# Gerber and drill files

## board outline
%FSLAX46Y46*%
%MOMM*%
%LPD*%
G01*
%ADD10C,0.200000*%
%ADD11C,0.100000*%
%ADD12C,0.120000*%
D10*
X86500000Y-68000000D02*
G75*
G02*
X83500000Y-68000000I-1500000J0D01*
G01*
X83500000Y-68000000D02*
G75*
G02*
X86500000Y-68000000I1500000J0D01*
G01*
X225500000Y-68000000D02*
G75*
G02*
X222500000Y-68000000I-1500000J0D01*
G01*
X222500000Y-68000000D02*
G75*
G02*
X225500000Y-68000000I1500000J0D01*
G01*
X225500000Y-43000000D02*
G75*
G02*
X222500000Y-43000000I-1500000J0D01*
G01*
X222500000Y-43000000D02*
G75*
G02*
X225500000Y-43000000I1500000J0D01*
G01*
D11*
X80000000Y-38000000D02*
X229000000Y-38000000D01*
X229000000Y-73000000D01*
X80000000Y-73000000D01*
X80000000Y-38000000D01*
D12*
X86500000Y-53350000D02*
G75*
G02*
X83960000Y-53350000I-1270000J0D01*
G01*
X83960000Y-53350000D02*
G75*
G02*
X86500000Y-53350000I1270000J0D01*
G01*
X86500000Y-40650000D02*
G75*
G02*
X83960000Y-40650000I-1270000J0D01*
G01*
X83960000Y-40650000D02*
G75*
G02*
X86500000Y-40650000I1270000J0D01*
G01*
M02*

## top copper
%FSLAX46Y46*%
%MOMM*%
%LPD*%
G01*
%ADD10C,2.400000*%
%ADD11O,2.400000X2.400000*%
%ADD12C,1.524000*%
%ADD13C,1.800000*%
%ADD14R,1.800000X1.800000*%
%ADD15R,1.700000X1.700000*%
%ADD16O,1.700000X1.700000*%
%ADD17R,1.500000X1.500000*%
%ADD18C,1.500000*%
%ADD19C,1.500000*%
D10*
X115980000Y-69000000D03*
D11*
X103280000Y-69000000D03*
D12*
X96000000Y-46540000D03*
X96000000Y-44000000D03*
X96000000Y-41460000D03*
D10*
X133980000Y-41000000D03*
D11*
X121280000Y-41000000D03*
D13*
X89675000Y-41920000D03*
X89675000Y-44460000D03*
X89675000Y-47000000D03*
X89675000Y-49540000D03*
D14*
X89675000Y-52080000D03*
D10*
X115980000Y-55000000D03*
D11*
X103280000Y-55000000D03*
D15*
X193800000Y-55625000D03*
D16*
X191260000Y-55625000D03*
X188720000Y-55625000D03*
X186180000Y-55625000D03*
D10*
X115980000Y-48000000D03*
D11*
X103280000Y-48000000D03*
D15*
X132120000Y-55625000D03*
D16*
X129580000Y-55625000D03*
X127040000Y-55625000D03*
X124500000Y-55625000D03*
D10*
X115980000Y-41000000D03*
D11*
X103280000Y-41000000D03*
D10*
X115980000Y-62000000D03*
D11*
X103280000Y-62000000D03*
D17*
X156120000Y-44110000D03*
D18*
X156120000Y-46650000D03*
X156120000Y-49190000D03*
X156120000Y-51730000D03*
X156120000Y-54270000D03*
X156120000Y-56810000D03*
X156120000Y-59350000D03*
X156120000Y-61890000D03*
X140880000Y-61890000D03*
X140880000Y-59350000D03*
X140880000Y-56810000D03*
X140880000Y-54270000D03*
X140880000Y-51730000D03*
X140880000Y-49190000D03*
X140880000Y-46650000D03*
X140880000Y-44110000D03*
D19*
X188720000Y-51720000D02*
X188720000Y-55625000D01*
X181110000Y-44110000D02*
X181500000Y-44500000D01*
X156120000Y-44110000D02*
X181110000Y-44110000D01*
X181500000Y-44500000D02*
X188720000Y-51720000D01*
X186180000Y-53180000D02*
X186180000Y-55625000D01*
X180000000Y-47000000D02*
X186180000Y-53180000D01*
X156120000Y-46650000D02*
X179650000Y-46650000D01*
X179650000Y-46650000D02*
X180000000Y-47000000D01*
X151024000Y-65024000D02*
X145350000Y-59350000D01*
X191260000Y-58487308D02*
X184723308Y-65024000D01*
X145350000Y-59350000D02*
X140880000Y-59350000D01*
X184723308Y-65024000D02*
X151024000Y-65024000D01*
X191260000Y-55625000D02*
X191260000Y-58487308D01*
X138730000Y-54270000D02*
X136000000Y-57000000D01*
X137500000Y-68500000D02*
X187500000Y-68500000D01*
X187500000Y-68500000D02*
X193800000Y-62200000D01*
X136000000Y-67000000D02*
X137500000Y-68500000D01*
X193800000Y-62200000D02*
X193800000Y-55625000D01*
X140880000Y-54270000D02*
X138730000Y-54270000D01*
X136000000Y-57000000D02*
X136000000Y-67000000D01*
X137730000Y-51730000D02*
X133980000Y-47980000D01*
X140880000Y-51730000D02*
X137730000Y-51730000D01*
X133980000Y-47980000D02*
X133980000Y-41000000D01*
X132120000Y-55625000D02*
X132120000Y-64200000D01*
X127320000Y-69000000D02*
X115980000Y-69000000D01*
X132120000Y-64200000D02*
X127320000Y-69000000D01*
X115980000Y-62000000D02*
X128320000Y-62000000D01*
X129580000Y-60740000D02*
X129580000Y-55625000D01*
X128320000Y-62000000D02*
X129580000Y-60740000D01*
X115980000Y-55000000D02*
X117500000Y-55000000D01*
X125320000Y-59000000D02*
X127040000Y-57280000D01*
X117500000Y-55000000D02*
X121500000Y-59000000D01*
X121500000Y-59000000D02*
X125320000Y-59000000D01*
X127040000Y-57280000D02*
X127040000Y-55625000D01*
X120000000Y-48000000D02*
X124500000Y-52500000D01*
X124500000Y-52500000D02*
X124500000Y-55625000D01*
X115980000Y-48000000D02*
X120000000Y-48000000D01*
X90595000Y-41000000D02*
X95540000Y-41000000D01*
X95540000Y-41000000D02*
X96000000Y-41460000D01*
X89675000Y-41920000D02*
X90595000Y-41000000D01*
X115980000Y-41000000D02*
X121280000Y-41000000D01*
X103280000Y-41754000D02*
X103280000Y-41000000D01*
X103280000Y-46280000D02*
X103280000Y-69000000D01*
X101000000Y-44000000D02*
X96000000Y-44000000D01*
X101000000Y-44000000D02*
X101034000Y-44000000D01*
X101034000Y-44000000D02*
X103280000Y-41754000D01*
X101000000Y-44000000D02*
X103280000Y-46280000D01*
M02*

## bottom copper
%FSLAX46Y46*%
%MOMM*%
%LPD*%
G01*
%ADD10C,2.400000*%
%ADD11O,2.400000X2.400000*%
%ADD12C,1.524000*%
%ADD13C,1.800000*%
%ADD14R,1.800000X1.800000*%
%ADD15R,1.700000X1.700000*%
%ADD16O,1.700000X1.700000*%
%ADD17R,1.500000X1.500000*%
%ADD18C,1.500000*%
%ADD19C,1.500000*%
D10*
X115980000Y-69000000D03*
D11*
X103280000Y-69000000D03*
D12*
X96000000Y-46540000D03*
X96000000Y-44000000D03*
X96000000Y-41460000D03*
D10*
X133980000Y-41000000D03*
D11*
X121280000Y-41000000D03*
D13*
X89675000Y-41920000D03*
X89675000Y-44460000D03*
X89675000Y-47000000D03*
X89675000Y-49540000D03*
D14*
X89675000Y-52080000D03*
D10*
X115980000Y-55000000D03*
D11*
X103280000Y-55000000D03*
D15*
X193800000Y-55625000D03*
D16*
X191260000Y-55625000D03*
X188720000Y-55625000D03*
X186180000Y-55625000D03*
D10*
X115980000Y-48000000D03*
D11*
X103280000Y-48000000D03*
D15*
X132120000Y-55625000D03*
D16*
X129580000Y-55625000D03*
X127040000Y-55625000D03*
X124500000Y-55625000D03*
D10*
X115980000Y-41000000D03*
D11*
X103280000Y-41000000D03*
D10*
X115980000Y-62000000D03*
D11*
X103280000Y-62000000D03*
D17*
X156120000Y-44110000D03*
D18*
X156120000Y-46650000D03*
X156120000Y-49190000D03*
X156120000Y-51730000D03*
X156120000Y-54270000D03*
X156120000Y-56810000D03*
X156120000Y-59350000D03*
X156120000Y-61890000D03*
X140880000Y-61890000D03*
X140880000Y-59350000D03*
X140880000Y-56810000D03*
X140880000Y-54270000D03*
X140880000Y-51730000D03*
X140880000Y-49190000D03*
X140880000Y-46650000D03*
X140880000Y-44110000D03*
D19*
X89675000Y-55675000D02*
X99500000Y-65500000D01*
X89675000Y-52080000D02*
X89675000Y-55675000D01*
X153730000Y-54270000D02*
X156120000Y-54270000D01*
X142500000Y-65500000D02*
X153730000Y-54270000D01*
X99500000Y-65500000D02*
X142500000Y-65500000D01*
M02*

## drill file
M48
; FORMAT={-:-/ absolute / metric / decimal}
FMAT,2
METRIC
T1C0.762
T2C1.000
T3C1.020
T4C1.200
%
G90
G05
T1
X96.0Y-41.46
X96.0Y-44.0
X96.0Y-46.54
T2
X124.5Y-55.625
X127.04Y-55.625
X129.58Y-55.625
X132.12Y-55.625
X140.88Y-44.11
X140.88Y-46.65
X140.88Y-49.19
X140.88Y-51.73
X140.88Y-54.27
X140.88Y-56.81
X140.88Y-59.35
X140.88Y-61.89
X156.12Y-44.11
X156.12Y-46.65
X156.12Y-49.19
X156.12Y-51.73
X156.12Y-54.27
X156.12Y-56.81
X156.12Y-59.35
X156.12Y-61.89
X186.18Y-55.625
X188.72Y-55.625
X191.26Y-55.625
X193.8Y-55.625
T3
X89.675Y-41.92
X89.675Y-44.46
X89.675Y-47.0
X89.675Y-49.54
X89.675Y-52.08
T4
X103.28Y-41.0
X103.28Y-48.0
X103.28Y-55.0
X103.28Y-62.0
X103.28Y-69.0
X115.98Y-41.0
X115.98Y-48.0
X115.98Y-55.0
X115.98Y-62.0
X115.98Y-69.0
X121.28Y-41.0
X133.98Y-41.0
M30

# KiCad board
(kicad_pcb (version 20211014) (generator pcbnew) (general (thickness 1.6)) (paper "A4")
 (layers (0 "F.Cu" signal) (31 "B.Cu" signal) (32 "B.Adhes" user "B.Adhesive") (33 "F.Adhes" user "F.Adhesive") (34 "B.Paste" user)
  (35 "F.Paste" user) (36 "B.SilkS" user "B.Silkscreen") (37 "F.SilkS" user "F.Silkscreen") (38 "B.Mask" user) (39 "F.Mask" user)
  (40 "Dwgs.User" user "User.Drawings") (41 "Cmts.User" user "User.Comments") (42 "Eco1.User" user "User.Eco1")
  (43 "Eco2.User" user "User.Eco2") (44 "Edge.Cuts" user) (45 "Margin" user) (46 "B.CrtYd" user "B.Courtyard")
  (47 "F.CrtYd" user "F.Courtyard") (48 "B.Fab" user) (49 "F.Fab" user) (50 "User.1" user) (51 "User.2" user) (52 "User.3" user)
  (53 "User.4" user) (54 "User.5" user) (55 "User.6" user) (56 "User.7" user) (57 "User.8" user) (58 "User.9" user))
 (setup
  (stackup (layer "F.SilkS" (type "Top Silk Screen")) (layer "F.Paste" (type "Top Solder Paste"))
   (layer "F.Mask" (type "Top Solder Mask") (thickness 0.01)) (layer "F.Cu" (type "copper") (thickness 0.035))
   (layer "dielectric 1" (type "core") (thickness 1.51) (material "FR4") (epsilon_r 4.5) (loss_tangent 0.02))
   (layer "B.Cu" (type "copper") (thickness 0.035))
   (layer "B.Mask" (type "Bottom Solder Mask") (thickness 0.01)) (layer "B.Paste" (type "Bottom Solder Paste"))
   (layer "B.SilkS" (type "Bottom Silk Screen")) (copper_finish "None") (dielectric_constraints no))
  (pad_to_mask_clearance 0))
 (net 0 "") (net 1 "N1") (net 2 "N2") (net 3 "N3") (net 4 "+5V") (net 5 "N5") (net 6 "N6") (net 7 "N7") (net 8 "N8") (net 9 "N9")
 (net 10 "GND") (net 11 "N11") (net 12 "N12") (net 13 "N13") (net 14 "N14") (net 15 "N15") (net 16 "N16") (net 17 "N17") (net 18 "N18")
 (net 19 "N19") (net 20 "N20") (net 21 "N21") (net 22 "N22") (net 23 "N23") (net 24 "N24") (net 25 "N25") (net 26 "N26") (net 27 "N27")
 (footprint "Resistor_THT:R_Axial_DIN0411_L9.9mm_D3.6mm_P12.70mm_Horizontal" (layer "F.Cu") (at 115.98 69 180)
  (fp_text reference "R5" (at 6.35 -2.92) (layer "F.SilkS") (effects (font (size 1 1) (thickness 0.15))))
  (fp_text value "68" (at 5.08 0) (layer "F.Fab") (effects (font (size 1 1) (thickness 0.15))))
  (pad "1" thru_hole circle (at 0 0 180) (size 2.4 2.4) (drill 1.2) (layers *.Cu *.Mask) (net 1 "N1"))
  (pad "2" thru_hole oval (at 12.7 0 180) (size 2.4 2.4) (drill 1.2) (layers *.Cu *.Mask) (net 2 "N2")))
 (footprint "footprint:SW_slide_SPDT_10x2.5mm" (layer "F.Cu") (at 96 44 90)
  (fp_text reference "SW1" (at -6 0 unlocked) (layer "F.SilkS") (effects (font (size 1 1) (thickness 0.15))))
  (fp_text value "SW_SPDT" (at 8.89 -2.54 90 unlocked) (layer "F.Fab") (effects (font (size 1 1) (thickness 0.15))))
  (pad "1" thru_hole circle (at -2.54 0 90) (size 1.524 1.524) (drill 0.762) (layers *.Cu *.Mask) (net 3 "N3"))
  (pad "2" thru_hole circle (at 0 0 90) (size 1.524 1.524) (drill 0.762) (layers *.Cu *.Mask) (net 2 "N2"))
  (pad "3" thru_hole circle (at 2.54 0 90) (size 1.524 1.524) (drill 0.762) (layers *.Cu *.Mask) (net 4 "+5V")))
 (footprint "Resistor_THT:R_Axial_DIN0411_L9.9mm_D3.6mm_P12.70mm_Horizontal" (layer "F.Cu") (at 133.98 41 180)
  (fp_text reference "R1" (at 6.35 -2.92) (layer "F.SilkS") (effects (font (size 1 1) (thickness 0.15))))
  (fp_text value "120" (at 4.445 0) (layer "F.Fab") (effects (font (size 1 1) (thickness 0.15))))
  (pad "1" thru_hole circle (at 0 0 180) (size 2.4 2.4) (drill 1.2) (layers *.Cu *.Mask) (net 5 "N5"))
  (pad "2" thru_hole oval (at 12.7 0 180) (size 2.4 2.4) (drill 1.2) (layers *.Cu *.Mask) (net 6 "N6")))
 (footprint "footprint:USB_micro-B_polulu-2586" (layer "F.Cu") (at 89.675 47 90)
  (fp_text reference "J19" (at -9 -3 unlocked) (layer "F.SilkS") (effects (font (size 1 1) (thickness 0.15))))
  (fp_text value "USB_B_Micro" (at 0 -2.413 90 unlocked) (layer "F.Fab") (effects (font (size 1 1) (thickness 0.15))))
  (fp_circle (center -6.35 -4.445) (end -7.62 -4.445) (layer "Edge.Cuts") (width 0.12) (fill none))
  (fp_circle (center 6.35 -4.445) (end 6.35 -5.715) (layer "Edge.Cuts") (width 0.12) (fill none))
  (pad "1" thru_hole circle (at 5.08 0 90) (size 1.8 1.8) (drill 1.02) (layers *.Cu *.Mask) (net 4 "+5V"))
  (pad "2" thru_hole circle (at 2.54 0 90) (size 1.8 1.8) (drill 1.02) (layers *.Cu *.Mask) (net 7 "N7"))
  (pad "3" thru_hole circle (at 0 0 90) (size 1.8 1.8) (drill 1.02) (layers *.Cu *.Mask) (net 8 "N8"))
  (pad "4" thru_hole circle (at -2.54 0 90) (size 1.8 1.8) (drill 1.02) (layers *.Cu *.Mask) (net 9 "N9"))
  (pad "5" thru_hole rect (at -5.08 0 90) (size 1.8 1.8) (drill 1.02) (layers *.Cu *.Mask) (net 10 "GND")))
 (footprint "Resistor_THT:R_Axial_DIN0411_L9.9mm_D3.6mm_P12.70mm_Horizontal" (layer "F.Cu") (at 115.98 55 180)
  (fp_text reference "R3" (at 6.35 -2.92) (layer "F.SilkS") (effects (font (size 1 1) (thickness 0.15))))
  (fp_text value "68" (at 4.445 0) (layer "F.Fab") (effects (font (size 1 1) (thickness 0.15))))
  (pad "1" thru_hole circle (at 0 0 180) (size 2.4 2.4) (drill 1.2) (layers *.Cu *.Mask) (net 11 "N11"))
  (pad "2" thru_hole oval (at 12.7 0 180) (size 2.4 2.4) (drill 1.2) (layers *.Cu *.Mask) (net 2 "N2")))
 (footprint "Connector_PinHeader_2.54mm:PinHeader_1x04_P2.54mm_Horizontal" (layer "F.Cu") (at 193.8 55.625 -90)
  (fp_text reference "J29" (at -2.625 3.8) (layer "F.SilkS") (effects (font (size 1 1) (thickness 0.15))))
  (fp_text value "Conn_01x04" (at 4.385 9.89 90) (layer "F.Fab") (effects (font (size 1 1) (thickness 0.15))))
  (pad "1" thru_hole rect (at 0 0 270) (size 1.7 1.7) (drill 1) (layers *.Cu *.Mask) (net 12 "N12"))
  (pad "2" thru_hole oval (at 0 2.54 270) (size 1.7 1.7) (drill 1) (layers *.Cu *.Mask) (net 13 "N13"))
  (pad "3" thru_hole oval (at 0 5.08 270) (size 1.7 1.7) (drill 1) (layers *.Cu *.Mask) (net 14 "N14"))
  (pad "4" thru_hole oval (at 0 7.62 270) (size 1.7 1.7) (drill 1) (layers *.Cu *.Mask) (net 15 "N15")))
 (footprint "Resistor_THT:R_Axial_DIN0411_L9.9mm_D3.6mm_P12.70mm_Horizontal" (layer "F.Cu") (at 115.98 48 180)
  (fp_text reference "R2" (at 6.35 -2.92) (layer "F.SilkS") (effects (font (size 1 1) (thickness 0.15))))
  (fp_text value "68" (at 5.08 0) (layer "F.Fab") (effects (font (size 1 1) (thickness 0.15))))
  (pad "1" thru_hole circle (at 0 0 180) (size 2.4 2.4) (drill 1.2) (layers *.Cu *.Mask) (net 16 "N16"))
  (pad "2" thru_hole oval (at 12.7 0 180) (size 2.4 2.4) (drill 1.2) (layers *.Cu *.Mask) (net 2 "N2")))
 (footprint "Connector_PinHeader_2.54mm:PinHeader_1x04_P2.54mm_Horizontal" (layer "F.Cu") (at 132.12 55.625 -90)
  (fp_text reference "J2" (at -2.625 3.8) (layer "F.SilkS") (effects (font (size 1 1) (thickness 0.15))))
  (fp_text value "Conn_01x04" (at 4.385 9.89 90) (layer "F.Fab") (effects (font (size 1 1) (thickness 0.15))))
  (pad "1" thru_hole rect (at 0 0 270) (size 1.7 1.7) (drill 1) (layers *.Cu *.Mask) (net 1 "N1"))
  (pad "2" thru_hole oval (at 0 2.54 270) (size 1.7 1.7) (drill 1) (layers *.Cu *.Mask) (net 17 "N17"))
  (pad "3" thru_hole oval (at 0 5.08 270) (size 1.7 1.7) (drill 1) (layers *.Cu *.Mask) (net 11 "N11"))
  (pad "4" thru_hole oval (at 0 7.62 270) (size 1.7 1.7) (drill 1) (layers *.Cu *.Mask) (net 16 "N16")))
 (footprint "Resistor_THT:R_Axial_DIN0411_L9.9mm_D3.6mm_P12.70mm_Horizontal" (layer "F.Cu") (at 115.98 41 180)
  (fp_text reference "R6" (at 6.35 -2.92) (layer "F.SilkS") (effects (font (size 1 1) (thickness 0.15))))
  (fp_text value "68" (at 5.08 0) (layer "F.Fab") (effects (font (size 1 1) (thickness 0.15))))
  (pad "1" thru_hole circle (at 0 0 180) (size 2.4 2.4) (drill 1.2) (layers *.Cu *.Mask) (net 6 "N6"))
  (pad "2" thru_hole oval (at 12.7 0 180) (size 2.4 2.4) (drill 1.2) (layers *.Cu *.Mask) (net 2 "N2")))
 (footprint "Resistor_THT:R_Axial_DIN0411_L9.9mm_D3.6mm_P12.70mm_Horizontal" (layer "F.Cu") (at 115.98 62 180)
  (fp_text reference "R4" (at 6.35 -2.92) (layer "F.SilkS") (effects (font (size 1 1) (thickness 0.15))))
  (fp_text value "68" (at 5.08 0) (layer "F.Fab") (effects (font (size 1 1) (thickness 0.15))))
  (pad "1" thru_hole circle (at 0 0 180) (size 2.4 2.4) (drill 1.2) (layers *.Cu *.Mask) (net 17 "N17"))
  (pad "2" thru_hole oval (at 12.7 0 180) (size 2.4 2.4) (drill 1.2) (layers *.Cu *.Mask) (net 2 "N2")))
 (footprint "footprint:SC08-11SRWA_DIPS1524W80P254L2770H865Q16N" (layer "B.Cu") (at 156.12 44.11 180)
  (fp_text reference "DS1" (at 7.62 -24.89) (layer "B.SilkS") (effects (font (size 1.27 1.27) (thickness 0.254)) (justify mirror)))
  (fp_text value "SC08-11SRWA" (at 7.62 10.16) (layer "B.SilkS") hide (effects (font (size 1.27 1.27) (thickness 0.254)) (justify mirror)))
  (pad "1" thru_hole rect (at 0 0 180) (size 1.5 1.5) (drill 1) (layers *.Cu *.Mask) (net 14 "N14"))
  (pad "2" thru_hole circle (at 0 -2.54 180) (size 1.5 1.5) (drill 1) (layers *.Cu *.Mask) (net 15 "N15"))
  (pad "3" thru_hole circle (at 0 -5.08 180) (size 1.5 1.5) (drill 1) (layers *.Cu *.Mask) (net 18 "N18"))
  (pad "4" thru_hole circle (at 0 -7.62 180) (size 1.5 1.5) (drill 1) (layers *.Cu *.Mask) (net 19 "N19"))
  (pad "5" thru_hole circle (at 0 -10.16 180) (size 1.5 1.5) (drill 1) (layers *.Cu *.Mask) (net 10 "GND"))
  (pad "6" thru_hole circle (at 0 -12.7 180) (size 1.5 1.5) (drill 1) (layers *.Cu *.Mask) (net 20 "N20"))
  (pad "7" thru_hole circle (at 0 -15.24 180) (size 1.5 1.5) (drill 1) (layers *.Cu *.Mask) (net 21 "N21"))
  (pad "8" thru_hole circle (at 0 -17.78 180) (size 1.5 1.5) (drill 1) (layers *.Cu *.Mask) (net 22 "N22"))
  (pad "9" thru_hole circle (at 15.24 -17.78 180) (size 1.5 1.5) (drill 1) (layers *.Cu *.Mask) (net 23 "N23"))
  (pad "10" thru_hole circle (at 15.24 -15.24 180) (size 1.5 1.5) (drill 1) (layers *.Cu *.Mask) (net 13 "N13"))
  (pad "11" thru_hole circle (at 15.24 -12.7 180) (size 1.5 1.5) (drill 1) (layers *.Cu *.Mask) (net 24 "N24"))
  (pad "12" thru_hole circle (at 15.24 -10.16 180) (size 1.5 1.5) (drill 1) (layers *.Cu *.Mask) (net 12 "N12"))
  (pad "13" thru_hole circle (at 15.24 -7.62 180) (size 1.5 1.5) (drill 1) (layers *.Cu *.Mask) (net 5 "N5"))
  (pad "14" thru_hole circle (at 15.24 -5.08 180) (size 1.5 1.5) (drill 1) (layers *.Cu *.Mask) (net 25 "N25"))
  (pad "15" thru_hole circle (at 15.24 -2.54 180) (size 1.5 1.5) (drill 1) (layers *.Cu *.Mask) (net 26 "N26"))
  (pad "16" thru_hole circle (at 15.24 0 180) (size 1.5 1.5) (drill 1) (layers *.Cu *.Mask) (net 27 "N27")))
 (gr_circle (center 85 68) (end 86.5 68) (layer "Edge.Cuts") (width 0.2) (fill none))
 (gr_circle (center 224 68) (end 225.5 68) (layer "Edge.Cuts") (width 0.2) (fill none))
 (gr_circle (center 224 43) (end 225.5 43) (layer "Edge.Cuts") (width 0.2) (fill none))
 (gr_rect (start 80 38) (end 229 73) (layer "Edge.Cuts") (width 0.1) (fill none))
 (segment (start 188.72 51.72) (end 188.72 55.625) (width 1.5) (layer "F.Cu") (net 14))
 (segment (start 181.11 44.11) (end 181.5 44.5) (width 1.5) (layer "F.Cu") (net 14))
 (segment (start 156.12 44.11) (end 181.11 44.11) (width 1.5) (layer "F.Cu") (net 14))
 (segment (start 181.5 44.5) (end 188.72 51.72) (width 1.5) (layer "F.Cu") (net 14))
 (segment (start 186.18 53.18) (end 186.18 55.625) (width 1.5) (layer "F.Cu") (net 15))
 (segment (start 180 47) (end 186.18 53.18) (width 1.5) (layer "F.Cu") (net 15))
 (segment (start 156.12 46.65) (end 179.65 46.65) (width 1.5) (layer "F.Cu") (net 15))
 (segment (start 179.65 46.65) (end 180 47) (width 1.5) (layer "F.Cu") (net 15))
 (segment (start 89.675 55.675) (end 99.5 65.5) (width 1.5) (layer "B.Cu") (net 10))
 (segment (start 89.675 52.08) (end 89.675 55.675) (width 1.5) (layer "B.Cu") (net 10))
 (segment (start 153.73 54.27) (end 156.12 54.27) (width 1.5) (layer "B.Cu") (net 10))
 (segment (start 142.5 65.5) (end 153.73 54.27) (width 1.5) (layer "B.Cu") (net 10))
 (segment (start 99.5 65.5) (end 142.5 65.5) (width 1.5) (layer "B.Cu") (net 10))
 (segment (start 151.024 65.024) (end 145.35 59.35) (width 1.5) (layer "F.Cu") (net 13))
 (segment (start 191.26 58.487308) (end 184.723308 65.024) (width 1.5) (layer "F.Cu") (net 13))
 (segment (start 145.35 59.35) (end 140.88 59.35) (width 1.5) (layer "F.Cu") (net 13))
 (segment (start 184.723308 65.024) (end 151.024 65.024) (width 1.5) (layer "F.Cu") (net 13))
 (segment (start 191.26 55.625) (end 191.26 58.487308) (width 1.5) (layer "F.Cu") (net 13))
 (segment (start 138.73 54.27) (end 136 57) (width 1.5) (layer "F.Cu") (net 12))
 (segment (start 137.5 68.5) (end 187.5 68.5) (width 1.5) (layer "F.Cu") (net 12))
 (segment (start 187.5 68.5) (end 193.8 62.2) (width 1.5) (layer "F.Cu") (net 12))
 (segment (start 136 67) (end 137.5 68.5) (width 1.5) (layer "F.Cu") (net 12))
 (segment (start 193.8 62.2) (end 193.8 55.625) (width 1.5) (layer "F.Cu") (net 12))
 (segment (start 140.88 54.27) (end 138.73 54.27) (width 1.5) (layer "F.Cu") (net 12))
 (segment (start 136 57) (end 136 67) (width 1.5) (layer "F.Cu") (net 12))
 (segment (start 137.73 51.73) (end 133.98 47.98) (width 1.5) (layer "F.Cu") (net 5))
 (segment (start 140.88 51.73) (end 137.73 51.73) (width 1.5) (layer "F.Cu") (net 5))
 (segment (start 133.98 47.98) (end 133.98 41) (width 1.5) (layer "F.Cu") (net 5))
 (segment (start 132.12 55.625) (end 132.12 64.2) (width 1.5) (layer "F.Cu") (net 1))
 (segment (start 127.32 69) (end 115.98 69) (width 1.5) (layer "F.Cu") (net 1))
 (segment (start 132.12 64.2) (end 127.32 69) (width 1.5) (layer "F.Cu") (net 1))
 (segment (start 115.98 62) (end 128.32 62) (width 1.5) (layer "F.Cu") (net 17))
 (segment (start 129.58 60.74) (end 129.58 55.625) (width 1.5) (layer "F.Cu") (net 17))
 (segment (start 128.32 62) (end 129.58 60.74) (width 1.5) (layer "F.Cu") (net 17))
 (segment (start 115.98 55) (end 117.5 55) (width 1.5) (layer "F.Cu") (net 11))
 (segment (start 125.32 59) (end 127.04 57.28) (width 1.5) (layer "F.Cu") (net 11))
 (segment (start 117.5 55) (end 121.5 59) (width 1.5) (layer "F.Cu") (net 11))
 (segment (start 121.5 59) (end 125.32 59) (width 1.5) (layer "F.Cu") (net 11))
 (segment (start 127.04 57.28) (end 127.04 55.625) (width 1.5) (layer "F.Cu") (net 11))
 (segment (start 120 48) (end 124.5 52.5) (width 1.5) (layer "F.Cu") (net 16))
 (segment (start 124.5 52.5) (end 124.5 55.625) (width 1.5) (layer "F.Cu") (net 16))
 (segment (start 115.98 48) (end 120 48) (width 1.5) (layer "F.Cu") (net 16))
 (segment (start 90.595 41) (end 95.54 41) (width 1.5) (layer "F.Cu") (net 4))
 (segment (start 95.54 41) (end 96 41.46) (width 1.5) (layer "F.Cu") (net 4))
 (segment (start 89.675 41.92) (end 90.595 41) (width 1.5) (layer "F.Cu") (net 4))
 (segment (start 115.98 41) (end 121.28 41) (width 1.5) (layer "F.Cu") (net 6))
 (segment (start 103.28 41.754) (end 103.28 41) (width 1.5) (layer "F.Cu") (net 2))
 (segment (start 103.28 46.28) (end 103.28 69) (width 1.5) (layer "F.Cu") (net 2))
 (segment (start 101 44) (end 96 44) (width 1.5) (layer "F.Cu") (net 2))
 (segment (start 101 44) (end 101.034 44) (width 1.5) (layer "F.Cu") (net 2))
 (segment (start 101.034 44) (end 103.28 41.754) (width 1.5) (layer "F.Cu") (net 2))
 (segment (start 101 44) (end 103.28 46.28) (width 1.5) (layer "F.Cu") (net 2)))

